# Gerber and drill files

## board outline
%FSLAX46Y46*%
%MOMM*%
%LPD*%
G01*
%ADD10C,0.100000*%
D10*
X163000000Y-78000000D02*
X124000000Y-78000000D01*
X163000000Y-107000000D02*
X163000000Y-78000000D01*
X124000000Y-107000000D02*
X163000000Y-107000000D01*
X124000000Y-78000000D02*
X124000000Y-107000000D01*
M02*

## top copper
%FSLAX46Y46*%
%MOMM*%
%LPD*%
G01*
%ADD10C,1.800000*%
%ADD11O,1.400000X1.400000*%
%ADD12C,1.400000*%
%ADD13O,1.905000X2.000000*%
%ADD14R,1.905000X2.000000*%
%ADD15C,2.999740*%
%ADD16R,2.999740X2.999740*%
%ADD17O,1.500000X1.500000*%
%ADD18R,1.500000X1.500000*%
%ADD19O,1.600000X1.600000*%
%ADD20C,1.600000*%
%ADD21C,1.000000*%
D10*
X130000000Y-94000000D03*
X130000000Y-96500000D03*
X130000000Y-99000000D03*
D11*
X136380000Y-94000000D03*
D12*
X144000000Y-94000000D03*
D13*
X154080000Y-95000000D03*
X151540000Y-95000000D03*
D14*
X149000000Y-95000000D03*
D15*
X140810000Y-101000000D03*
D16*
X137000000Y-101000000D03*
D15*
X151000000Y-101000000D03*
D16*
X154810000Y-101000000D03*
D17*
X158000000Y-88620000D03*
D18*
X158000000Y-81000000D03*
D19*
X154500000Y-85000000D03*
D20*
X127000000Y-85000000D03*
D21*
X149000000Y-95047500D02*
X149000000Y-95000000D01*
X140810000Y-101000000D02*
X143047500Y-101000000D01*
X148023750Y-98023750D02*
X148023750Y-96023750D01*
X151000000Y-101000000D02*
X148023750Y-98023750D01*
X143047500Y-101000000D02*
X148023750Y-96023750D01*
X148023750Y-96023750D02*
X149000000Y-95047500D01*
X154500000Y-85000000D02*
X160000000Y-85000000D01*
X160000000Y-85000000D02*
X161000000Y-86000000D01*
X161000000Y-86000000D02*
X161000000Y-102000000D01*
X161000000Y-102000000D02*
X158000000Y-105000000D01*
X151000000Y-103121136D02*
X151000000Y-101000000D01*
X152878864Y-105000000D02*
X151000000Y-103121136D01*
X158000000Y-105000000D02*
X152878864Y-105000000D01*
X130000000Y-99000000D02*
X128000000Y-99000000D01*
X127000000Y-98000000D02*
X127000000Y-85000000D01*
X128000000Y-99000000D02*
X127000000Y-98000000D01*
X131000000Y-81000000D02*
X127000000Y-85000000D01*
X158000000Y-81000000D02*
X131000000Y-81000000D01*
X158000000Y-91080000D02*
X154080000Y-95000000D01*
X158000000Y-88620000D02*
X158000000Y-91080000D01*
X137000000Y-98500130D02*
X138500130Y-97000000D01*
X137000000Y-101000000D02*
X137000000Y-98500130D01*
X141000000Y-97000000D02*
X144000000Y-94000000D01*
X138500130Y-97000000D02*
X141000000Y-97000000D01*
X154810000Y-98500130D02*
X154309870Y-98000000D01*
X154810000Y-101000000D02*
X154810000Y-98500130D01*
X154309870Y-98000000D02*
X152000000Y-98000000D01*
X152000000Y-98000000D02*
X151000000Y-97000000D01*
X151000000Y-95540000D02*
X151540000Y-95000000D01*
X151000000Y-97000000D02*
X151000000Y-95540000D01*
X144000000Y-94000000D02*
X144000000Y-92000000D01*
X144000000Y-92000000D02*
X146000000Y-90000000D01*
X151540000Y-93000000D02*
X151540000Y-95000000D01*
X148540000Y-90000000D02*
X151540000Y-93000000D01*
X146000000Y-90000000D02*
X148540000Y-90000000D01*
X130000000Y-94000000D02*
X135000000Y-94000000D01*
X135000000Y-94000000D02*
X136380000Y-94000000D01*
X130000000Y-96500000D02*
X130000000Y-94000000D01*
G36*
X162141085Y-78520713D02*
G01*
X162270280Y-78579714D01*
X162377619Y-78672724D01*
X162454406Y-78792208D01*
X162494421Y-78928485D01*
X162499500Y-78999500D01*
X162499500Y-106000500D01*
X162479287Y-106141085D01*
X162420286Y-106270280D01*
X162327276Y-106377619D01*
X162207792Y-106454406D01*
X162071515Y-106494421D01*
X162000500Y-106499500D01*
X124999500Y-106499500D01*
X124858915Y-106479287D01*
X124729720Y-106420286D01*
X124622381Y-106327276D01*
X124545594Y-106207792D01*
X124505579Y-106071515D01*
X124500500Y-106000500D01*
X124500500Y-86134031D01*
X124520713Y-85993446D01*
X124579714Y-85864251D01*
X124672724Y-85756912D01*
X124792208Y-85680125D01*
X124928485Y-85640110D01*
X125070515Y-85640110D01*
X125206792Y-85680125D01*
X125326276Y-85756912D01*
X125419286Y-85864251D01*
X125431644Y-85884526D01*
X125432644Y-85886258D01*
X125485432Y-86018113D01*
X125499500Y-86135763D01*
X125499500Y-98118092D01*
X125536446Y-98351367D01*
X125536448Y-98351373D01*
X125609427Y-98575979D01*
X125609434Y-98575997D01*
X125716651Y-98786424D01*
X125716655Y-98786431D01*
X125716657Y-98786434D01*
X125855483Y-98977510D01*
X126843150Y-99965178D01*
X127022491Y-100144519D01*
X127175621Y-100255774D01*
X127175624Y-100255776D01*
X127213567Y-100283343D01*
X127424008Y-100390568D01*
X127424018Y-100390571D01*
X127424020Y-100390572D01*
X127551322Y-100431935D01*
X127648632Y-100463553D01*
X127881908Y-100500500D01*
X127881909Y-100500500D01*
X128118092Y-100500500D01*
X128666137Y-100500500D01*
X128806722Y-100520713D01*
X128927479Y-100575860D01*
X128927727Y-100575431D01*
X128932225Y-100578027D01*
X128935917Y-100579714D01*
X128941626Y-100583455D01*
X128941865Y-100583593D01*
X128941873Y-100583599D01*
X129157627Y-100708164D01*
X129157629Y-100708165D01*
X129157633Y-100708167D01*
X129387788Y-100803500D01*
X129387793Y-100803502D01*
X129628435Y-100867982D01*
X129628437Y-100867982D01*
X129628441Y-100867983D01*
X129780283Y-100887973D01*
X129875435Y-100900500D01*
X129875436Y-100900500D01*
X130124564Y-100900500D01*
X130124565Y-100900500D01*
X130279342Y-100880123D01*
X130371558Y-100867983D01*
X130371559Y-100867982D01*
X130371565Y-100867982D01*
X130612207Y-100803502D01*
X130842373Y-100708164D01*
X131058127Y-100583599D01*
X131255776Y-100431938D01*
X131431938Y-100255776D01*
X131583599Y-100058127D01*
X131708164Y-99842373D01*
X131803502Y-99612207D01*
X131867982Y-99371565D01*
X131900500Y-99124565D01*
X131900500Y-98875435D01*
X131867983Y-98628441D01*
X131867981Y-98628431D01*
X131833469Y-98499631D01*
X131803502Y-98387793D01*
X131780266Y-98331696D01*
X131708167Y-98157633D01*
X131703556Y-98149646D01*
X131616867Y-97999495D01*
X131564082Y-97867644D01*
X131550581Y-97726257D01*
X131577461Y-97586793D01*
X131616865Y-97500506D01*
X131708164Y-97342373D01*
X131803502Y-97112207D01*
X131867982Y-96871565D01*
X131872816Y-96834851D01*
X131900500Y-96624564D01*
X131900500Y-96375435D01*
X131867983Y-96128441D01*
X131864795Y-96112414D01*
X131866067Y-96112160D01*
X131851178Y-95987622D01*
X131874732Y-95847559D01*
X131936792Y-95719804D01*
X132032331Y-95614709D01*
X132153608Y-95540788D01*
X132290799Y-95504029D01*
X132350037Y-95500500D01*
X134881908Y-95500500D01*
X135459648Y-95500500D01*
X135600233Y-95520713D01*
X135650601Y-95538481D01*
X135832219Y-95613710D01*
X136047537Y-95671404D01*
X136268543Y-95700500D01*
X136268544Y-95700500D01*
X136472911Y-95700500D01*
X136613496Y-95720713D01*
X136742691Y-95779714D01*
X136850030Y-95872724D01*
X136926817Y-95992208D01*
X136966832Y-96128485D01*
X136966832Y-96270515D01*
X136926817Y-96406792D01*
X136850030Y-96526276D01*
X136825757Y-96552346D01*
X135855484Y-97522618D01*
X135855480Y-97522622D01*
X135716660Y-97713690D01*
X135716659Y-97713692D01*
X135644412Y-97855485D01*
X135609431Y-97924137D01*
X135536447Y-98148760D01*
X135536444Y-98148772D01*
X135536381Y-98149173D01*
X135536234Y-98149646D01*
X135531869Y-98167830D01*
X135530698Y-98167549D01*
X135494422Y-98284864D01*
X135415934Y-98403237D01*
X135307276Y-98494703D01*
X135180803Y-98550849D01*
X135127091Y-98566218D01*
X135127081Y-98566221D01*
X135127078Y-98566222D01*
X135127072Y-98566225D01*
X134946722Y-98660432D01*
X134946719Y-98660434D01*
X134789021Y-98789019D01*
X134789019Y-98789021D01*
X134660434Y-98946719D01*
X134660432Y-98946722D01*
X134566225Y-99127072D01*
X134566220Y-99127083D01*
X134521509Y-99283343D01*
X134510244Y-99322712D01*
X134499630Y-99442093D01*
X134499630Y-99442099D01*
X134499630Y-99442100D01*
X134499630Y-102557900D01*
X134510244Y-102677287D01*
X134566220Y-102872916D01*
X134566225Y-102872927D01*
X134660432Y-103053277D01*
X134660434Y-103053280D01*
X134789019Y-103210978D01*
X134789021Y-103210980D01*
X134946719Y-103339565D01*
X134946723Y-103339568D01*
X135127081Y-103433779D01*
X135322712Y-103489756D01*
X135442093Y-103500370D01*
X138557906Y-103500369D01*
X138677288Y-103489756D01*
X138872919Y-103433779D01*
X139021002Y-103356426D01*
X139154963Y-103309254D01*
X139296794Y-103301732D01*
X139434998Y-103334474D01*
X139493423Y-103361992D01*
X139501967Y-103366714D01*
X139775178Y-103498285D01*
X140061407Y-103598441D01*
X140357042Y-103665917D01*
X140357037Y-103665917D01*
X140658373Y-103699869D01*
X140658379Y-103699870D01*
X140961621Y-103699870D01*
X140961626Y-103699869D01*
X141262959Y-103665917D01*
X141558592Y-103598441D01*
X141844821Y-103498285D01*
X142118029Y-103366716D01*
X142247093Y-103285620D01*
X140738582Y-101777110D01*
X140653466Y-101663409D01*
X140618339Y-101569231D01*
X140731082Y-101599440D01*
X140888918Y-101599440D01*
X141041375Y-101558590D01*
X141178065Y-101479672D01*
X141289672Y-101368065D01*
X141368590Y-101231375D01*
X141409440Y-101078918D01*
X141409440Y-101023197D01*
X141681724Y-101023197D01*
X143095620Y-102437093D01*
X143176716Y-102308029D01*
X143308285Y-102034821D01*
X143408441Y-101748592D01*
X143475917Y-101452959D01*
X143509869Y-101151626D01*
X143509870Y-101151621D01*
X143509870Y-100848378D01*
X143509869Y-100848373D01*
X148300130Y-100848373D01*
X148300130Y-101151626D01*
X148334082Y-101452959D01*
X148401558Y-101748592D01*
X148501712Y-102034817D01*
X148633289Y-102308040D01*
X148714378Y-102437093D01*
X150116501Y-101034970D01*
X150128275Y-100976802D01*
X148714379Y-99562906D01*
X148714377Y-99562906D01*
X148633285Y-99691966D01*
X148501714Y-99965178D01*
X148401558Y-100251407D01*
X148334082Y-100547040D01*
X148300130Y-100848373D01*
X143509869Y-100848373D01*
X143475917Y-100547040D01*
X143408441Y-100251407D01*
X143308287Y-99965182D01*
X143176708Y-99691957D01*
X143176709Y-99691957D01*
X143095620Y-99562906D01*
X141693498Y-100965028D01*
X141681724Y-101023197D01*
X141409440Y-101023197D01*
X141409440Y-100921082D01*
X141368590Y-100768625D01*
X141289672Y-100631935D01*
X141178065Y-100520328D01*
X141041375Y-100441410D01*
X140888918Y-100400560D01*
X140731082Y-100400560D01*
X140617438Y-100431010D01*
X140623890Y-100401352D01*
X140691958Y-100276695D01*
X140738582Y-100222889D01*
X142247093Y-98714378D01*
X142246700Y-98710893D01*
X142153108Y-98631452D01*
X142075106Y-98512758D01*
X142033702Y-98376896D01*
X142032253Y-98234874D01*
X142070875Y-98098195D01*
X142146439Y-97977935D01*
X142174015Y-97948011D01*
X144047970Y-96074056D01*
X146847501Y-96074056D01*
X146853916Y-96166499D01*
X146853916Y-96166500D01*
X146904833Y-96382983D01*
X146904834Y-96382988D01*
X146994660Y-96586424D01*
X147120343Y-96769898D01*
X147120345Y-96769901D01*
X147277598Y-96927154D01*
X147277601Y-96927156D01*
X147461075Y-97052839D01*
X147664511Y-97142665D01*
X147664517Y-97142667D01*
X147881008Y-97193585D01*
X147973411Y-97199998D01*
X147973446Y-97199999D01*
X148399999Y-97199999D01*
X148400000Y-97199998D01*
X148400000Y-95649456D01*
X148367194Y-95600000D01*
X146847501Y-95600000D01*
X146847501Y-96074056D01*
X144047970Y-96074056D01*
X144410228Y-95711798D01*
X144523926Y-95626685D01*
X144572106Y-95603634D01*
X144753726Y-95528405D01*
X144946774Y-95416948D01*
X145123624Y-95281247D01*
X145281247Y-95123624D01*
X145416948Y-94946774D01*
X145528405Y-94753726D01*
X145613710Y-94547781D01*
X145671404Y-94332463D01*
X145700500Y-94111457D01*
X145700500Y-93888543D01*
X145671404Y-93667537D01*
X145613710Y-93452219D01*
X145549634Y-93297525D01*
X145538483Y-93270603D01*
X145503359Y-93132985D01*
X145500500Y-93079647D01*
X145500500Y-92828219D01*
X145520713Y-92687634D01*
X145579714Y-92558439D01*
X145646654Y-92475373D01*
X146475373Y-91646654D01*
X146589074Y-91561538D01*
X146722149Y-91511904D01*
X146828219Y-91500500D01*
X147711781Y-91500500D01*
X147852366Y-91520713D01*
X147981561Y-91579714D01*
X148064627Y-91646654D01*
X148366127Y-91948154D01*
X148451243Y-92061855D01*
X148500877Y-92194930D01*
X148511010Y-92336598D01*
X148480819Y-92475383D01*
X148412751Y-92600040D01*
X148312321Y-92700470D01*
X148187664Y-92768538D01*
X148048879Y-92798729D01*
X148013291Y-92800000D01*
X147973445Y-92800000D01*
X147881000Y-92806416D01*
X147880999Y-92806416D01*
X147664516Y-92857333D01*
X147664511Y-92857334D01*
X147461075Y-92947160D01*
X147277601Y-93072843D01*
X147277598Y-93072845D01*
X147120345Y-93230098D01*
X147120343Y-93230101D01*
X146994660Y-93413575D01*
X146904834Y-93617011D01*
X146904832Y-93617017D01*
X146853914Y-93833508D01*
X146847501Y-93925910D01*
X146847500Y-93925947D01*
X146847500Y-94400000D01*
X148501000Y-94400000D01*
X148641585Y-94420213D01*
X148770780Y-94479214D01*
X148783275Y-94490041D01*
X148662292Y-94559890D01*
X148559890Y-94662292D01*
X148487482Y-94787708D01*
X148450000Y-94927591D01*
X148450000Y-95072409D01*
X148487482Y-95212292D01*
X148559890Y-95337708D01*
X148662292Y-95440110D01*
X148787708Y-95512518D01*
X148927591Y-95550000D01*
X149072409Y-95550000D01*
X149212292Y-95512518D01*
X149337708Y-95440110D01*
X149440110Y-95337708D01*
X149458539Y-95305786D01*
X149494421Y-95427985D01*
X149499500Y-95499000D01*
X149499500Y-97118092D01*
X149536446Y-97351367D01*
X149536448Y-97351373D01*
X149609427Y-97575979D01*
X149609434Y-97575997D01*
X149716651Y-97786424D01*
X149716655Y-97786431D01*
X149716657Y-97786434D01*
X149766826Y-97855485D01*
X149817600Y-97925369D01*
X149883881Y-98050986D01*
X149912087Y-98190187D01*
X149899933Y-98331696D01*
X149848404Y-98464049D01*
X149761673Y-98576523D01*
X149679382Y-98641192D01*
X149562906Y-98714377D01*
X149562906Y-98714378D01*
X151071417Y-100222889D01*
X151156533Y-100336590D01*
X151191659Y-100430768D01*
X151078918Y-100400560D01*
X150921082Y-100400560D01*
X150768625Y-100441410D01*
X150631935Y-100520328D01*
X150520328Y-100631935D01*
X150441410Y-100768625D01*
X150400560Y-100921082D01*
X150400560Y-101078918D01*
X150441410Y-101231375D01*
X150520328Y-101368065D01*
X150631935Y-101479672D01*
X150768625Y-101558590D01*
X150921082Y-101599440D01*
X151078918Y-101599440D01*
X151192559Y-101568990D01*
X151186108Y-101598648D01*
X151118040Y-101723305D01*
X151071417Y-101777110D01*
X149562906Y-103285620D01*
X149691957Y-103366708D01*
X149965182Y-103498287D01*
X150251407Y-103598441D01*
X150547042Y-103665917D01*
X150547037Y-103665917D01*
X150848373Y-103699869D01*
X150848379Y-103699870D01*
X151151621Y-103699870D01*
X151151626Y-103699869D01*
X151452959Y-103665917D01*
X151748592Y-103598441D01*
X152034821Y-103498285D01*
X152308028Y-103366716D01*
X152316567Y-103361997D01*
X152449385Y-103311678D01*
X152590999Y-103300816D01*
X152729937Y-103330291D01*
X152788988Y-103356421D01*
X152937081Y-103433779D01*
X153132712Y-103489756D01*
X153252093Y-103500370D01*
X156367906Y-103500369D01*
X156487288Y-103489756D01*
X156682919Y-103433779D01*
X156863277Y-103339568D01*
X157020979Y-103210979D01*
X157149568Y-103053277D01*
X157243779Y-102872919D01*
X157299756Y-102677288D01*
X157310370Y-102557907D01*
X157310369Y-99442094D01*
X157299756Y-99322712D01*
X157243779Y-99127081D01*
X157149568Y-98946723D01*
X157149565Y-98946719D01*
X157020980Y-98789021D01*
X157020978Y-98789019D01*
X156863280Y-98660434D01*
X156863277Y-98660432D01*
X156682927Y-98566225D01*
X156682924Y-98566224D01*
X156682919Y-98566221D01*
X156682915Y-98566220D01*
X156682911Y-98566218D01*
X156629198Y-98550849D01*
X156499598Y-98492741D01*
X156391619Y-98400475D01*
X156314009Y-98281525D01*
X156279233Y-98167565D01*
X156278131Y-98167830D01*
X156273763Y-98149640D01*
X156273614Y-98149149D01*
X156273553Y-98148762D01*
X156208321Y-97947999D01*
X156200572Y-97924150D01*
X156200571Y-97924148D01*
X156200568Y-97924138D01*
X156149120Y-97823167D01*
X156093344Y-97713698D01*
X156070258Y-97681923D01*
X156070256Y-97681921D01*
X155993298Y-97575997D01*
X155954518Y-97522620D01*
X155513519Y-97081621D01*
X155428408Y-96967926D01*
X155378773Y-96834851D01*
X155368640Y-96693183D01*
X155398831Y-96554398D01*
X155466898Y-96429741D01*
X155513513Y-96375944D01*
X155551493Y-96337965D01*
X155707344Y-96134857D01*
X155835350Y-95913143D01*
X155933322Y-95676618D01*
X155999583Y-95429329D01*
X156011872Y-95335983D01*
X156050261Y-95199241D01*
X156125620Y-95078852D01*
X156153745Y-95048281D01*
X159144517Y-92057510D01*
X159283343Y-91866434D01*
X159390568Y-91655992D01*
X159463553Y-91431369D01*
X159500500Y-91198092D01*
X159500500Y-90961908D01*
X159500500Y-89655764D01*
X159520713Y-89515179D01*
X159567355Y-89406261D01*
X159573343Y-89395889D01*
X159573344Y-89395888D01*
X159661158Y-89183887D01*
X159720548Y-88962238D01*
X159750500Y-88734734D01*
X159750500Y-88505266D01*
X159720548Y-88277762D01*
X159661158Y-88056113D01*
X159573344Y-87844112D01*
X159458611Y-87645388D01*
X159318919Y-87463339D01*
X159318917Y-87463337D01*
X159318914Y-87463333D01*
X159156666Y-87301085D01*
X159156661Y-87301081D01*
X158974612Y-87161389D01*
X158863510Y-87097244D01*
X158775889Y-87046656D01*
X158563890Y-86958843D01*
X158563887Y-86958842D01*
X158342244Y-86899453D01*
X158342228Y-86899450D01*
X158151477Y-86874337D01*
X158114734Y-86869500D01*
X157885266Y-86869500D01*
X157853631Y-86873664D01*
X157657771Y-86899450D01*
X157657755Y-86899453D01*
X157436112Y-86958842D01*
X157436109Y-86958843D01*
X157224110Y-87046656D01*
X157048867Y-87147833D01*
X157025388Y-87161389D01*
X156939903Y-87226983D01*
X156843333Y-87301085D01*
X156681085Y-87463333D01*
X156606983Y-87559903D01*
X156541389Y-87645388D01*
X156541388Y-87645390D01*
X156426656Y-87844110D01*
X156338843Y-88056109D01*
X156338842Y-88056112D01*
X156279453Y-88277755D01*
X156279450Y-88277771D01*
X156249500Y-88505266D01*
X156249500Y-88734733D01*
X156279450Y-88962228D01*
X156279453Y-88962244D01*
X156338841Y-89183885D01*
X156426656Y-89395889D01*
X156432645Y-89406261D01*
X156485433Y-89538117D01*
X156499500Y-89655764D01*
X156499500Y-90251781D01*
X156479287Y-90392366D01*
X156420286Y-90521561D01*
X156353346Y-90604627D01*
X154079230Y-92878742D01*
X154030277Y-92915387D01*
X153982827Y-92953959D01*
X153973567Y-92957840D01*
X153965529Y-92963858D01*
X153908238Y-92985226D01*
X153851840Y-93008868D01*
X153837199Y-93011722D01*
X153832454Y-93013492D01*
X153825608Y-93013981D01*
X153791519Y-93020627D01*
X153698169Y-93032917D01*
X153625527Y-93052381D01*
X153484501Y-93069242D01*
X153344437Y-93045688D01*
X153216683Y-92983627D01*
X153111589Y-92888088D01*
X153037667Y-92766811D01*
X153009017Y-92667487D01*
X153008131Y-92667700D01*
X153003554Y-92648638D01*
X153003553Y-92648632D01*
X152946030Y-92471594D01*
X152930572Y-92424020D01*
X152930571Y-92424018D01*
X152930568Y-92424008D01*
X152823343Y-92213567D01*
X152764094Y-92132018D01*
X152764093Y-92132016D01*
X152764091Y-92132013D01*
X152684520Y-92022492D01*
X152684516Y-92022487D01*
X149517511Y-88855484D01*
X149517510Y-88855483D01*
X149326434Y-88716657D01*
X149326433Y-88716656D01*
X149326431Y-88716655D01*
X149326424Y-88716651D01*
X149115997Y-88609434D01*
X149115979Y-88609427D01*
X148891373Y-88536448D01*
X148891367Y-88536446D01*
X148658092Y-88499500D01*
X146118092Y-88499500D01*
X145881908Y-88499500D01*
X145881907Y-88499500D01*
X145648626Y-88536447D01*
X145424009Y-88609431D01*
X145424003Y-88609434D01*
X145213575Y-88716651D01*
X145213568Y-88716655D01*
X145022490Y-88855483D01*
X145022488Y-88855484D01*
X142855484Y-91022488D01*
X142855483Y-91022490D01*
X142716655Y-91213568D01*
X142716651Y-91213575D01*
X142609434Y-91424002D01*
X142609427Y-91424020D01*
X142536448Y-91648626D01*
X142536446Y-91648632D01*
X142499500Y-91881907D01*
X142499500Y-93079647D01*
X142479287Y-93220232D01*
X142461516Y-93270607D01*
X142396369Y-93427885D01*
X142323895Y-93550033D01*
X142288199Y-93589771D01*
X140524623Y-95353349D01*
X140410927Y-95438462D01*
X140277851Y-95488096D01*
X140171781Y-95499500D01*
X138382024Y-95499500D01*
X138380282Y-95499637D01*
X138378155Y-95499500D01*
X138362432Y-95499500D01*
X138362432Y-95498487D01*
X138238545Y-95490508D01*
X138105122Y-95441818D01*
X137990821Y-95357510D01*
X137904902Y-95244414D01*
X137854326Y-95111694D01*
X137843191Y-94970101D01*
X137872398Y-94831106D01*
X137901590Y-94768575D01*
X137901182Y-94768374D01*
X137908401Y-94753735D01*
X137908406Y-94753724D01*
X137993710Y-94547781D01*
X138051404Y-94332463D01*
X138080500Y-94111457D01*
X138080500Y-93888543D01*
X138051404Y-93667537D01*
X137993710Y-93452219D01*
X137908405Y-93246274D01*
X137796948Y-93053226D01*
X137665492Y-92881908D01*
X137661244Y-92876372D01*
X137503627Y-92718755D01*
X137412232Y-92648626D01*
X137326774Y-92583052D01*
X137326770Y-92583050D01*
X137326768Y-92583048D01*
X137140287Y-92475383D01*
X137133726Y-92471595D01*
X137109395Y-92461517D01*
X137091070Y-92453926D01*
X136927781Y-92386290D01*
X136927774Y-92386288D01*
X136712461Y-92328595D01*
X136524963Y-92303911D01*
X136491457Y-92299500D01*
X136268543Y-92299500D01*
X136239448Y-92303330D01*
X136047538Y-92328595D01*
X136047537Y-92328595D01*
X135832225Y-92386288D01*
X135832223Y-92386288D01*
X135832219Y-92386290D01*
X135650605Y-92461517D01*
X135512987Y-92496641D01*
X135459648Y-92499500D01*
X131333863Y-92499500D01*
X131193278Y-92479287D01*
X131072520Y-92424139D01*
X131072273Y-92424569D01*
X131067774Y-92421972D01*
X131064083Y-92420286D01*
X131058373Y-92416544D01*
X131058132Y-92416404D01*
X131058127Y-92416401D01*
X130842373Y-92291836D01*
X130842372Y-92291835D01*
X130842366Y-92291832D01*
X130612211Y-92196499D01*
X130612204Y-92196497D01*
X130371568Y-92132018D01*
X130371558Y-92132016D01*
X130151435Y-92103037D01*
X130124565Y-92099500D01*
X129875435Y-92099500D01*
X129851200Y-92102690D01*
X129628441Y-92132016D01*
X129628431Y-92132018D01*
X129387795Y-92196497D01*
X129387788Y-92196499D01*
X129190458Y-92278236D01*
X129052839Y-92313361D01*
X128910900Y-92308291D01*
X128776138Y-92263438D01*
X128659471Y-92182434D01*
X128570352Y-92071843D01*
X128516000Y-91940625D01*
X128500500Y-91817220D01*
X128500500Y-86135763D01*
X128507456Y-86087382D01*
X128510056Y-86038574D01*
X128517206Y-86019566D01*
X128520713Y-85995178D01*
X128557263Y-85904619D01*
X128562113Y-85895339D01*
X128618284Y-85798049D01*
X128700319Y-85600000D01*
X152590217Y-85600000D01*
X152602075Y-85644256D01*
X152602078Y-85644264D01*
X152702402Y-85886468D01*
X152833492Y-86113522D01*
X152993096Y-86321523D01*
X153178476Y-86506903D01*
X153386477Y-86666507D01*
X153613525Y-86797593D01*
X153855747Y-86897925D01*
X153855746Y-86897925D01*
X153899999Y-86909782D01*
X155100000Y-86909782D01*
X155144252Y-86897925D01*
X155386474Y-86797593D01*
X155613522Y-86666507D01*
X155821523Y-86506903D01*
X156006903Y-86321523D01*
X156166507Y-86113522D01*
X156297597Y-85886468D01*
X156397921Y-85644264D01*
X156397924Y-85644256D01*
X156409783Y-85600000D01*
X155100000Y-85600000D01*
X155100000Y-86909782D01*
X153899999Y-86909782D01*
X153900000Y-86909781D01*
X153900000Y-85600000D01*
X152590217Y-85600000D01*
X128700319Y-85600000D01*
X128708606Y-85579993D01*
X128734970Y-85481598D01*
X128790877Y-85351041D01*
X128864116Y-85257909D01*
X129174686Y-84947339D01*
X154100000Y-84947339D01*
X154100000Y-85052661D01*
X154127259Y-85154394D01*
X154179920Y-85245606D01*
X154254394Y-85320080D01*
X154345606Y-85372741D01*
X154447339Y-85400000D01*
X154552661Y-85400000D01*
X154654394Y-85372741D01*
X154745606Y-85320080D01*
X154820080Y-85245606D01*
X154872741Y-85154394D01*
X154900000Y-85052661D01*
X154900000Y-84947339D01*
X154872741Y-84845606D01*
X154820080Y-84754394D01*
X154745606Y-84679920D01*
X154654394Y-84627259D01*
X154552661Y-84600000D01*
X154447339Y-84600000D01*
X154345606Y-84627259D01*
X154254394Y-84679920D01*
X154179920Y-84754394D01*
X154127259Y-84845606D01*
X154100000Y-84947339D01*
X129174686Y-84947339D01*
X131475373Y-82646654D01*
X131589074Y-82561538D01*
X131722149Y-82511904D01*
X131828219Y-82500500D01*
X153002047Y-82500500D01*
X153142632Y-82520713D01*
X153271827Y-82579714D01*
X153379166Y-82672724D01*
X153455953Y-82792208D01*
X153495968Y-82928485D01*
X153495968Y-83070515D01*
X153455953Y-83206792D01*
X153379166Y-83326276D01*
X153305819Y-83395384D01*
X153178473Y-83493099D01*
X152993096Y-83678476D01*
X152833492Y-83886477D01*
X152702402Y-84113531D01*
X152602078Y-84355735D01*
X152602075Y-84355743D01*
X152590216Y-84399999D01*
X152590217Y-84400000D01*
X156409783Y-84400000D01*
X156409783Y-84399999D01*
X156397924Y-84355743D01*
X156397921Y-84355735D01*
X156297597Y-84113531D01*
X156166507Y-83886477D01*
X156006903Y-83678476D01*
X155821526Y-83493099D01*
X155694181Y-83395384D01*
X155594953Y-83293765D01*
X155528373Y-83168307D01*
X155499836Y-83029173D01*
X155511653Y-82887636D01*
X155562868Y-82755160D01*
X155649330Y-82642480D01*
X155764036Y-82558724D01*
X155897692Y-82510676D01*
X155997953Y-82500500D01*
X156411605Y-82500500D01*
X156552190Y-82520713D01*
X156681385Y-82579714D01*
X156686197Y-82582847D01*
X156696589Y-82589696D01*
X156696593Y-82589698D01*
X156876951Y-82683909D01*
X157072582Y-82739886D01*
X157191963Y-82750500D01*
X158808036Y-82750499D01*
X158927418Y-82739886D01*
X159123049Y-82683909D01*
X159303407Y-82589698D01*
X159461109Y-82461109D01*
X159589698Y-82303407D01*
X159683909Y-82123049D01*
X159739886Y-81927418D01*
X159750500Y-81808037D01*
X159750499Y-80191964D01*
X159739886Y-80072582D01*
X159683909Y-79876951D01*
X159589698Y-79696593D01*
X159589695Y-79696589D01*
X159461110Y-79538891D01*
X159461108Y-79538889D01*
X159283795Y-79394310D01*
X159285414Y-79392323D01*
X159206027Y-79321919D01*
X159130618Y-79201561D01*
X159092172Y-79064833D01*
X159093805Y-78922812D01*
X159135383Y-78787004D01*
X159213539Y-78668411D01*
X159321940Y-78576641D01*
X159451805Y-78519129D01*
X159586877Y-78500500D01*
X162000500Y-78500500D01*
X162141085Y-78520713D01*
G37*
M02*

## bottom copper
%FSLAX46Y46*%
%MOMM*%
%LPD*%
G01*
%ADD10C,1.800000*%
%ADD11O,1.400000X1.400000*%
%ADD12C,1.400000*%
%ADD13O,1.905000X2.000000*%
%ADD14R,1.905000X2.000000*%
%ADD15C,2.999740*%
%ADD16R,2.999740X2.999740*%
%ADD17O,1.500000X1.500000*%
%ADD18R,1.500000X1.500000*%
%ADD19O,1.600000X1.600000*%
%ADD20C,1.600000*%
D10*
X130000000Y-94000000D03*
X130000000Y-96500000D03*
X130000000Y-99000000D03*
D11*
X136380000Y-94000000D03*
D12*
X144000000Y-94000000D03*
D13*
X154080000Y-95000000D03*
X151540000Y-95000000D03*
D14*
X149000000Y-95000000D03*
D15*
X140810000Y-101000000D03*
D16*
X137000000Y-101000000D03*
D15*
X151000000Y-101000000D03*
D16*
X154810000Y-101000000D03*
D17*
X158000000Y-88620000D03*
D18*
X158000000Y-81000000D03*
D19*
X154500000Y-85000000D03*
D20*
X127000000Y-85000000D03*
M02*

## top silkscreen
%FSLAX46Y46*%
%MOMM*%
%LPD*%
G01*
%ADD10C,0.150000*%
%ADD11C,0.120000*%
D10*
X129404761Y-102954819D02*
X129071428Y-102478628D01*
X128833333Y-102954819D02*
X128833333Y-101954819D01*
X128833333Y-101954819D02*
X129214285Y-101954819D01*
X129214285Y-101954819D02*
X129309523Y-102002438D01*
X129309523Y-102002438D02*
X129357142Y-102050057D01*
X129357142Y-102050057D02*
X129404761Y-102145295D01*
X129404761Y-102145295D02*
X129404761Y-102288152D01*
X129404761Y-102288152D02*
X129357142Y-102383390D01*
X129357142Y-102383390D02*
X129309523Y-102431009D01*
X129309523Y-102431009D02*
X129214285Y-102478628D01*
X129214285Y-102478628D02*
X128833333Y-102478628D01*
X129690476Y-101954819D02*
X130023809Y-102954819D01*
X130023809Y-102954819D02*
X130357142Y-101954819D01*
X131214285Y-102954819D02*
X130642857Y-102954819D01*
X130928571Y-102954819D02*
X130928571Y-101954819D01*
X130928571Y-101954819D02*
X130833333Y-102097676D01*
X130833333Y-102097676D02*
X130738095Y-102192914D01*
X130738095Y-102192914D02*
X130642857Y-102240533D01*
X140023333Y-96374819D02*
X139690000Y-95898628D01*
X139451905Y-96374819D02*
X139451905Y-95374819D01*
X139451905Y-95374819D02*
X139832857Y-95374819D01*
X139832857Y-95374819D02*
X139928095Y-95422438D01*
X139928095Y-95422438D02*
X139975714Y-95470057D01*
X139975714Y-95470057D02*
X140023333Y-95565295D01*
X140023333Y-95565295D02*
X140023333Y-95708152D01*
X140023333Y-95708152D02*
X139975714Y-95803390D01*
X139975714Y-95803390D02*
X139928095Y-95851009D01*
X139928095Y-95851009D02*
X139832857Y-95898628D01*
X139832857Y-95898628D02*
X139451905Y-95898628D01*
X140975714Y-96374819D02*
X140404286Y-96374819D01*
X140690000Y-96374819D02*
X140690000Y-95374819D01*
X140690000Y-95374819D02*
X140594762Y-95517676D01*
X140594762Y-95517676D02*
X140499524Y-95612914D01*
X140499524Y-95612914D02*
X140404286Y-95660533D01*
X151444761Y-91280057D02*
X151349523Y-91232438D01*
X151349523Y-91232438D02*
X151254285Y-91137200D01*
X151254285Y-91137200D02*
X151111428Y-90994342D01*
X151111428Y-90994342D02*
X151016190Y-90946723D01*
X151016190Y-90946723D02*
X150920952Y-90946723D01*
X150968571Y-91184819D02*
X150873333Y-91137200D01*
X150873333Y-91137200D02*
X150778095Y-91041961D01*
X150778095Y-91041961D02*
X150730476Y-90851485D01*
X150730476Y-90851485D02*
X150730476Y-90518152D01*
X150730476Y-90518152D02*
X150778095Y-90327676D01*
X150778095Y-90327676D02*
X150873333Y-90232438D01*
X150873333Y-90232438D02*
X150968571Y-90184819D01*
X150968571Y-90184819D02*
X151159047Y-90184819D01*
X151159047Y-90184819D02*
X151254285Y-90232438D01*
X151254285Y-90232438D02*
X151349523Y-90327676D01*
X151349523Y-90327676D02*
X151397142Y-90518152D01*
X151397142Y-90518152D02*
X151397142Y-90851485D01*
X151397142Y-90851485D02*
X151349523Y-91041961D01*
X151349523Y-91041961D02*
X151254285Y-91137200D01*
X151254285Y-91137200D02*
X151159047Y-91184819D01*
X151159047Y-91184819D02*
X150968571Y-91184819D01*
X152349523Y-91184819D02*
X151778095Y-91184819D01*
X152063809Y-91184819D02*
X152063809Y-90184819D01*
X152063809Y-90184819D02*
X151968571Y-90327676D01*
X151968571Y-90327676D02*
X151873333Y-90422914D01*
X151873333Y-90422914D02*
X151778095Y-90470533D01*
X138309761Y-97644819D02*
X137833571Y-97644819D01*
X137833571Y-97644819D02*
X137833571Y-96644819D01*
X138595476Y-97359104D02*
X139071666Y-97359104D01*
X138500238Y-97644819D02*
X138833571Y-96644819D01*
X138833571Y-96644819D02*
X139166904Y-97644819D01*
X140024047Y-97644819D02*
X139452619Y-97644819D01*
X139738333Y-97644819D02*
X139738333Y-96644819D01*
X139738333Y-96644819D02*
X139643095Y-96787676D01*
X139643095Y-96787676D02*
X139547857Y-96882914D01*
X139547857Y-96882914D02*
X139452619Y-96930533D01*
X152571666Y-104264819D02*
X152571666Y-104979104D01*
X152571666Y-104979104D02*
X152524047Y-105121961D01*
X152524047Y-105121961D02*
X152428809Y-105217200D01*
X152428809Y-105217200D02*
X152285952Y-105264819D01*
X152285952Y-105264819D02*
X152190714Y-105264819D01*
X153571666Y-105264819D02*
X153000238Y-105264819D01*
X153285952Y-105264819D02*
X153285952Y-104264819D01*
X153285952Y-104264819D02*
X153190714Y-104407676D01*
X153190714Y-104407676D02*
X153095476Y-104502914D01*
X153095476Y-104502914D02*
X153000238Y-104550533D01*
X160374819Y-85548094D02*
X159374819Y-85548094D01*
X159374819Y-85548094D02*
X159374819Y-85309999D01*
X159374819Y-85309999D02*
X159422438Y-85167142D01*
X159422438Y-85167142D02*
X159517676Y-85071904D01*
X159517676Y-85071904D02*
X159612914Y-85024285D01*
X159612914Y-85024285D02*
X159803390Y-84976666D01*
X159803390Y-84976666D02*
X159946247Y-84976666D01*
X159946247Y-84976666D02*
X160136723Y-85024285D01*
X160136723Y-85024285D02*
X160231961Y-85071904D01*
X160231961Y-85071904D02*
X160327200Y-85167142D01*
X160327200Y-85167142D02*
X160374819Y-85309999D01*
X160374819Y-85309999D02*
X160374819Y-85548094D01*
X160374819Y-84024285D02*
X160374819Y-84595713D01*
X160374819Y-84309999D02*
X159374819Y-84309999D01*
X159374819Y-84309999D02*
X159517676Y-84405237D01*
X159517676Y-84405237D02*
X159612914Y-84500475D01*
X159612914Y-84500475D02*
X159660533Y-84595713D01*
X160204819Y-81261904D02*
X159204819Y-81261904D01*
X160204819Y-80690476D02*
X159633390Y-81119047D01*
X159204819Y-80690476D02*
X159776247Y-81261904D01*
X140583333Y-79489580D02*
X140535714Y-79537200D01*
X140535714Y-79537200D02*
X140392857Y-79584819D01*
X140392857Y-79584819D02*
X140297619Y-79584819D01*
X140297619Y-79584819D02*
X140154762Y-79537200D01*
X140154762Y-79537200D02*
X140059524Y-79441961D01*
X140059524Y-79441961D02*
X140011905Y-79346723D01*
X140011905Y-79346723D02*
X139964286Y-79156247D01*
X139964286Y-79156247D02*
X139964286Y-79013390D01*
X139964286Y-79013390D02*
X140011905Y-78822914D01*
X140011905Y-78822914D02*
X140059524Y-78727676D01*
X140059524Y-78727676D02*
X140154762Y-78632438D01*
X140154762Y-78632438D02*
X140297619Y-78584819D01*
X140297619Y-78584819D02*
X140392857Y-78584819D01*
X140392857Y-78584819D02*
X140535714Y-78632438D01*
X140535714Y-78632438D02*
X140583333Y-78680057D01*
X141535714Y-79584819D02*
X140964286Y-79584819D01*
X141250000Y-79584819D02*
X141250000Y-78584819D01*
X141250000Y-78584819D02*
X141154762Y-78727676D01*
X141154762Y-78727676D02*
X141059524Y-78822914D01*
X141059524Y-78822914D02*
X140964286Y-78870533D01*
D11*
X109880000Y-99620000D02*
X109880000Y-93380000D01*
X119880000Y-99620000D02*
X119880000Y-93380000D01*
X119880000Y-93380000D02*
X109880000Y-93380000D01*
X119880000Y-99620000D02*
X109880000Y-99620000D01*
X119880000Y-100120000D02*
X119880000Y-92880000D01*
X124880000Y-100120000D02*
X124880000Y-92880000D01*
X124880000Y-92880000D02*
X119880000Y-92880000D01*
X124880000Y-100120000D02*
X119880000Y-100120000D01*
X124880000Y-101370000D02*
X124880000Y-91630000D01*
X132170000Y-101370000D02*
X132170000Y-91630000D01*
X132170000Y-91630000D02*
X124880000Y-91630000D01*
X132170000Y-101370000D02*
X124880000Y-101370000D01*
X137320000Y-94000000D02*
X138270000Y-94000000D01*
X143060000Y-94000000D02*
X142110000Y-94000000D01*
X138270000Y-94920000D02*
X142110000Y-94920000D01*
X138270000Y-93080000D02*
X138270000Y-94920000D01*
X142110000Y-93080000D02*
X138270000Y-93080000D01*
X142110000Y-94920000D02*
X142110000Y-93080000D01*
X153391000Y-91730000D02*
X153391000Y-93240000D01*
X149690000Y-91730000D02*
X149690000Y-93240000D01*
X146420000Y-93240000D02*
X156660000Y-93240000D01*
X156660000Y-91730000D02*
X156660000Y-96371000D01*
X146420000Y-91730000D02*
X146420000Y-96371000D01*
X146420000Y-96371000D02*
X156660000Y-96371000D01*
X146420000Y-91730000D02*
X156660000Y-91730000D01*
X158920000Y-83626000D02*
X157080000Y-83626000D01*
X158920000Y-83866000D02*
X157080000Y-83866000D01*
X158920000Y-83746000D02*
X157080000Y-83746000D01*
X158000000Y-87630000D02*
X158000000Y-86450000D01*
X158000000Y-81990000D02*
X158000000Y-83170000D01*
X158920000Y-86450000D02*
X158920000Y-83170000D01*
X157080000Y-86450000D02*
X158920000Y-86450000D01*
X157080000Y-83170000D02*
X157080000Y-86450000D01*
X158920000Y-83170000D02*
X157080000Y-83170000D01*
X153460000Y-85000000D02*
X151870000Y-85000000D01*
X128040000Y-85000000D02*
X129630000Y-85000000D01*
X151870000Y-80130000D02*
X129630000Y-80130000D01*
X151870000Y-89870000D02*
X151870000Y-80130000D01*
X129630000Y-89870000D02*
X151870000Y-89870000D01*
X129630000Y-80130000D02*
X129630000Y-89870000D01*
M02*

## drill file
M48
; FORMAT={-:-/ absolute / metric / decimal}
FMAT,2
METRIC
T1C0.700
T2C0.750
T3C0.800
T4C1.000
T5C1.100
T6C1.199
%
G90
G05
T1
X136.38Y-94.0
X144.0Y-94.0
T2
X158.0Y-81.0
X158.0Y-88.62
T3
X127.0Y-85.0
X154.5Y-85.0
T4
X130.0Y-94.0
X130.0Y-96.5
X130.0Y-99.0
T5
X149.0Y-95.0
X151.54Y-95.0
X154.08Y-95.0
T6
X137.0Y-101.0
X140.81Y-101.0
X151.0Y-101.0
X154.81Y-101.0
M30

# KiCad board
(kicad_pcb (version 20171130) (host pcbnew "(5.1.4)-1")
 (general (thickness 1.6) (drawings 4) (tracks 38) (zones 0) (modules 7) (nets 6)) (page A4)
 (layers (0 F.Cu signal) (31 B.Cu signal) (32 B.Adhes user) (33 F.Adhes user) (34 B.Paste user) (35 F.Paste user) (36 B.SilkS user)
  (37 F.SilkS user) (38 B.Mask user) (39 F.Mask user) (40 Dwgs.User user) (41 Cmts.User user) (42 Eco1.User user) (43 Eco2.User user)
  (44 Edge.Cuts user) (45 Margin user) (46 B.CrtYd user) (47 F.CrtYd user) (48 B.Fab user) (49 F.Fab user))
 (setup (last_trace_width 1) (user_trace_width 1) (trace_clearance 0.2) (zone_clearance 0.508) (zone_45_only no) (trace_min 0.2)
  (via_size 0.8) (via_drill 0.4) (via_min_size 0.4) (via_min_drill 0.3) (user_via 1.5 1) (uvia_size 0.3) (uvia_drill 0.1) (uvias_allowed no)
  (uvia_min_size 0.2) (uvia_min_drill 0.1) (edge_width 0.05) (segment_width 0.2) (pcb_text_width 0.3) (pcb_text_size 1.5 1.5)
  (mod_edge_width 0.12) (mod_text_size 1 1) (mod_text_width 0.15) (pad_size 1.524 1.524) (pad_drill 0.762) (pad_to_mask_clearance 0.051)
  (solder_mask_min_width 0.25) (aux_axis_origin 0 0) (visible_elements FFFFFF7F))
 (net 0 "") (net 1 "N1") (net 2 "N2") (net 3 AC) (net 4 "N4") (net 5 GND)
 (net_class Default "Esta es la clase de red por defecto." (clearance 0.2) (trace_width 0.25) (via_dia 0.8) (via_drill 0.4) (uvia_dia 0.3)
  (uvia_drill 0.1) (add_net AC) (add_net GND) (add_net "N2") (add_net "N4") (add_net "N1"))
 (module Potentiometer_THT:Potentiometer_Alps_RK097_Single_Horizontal (layer F.Cu) (at 130 94 180)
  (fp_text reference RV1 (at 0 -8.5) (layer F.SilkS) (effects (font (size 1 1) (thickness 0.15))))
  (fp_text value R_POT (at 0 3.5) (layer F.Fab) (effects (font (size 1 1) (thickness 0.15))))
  (fp_line (start 20.12 -5.62) (end 20.12 0.62) (layer F.SilkS) (width 0.12))
  (fp_line (start 10.12 -5.62) (end 10.12 0.62) (layer F.SilkS) (width 0.12))
  (fp_line (start 10.12 0.62) (end 20.12 0.62) (layer F.SilkS) (width 0.12))
  (fp_line (start 10.12 -5.62) (end 20.12 -5.62) (layer F.SilkS) (width 0.12))
  (fp_line (start 10.12 -6.12) (end 10.12 1.12) (layer F.SilkS) (width 0.12))
  (fp_line (start 5.12 -6.12) (end 5.12 1.12) (layer F.SilkS) (width 0.12))
  (fp_line (start 5.12 1.12) (end 10.12 1.12) (layer F.SilkS) (width 0.12))
  (fp_line (start 5.12 -6.12) (end 10.12 -6.12) (layer F.SilkS) (width 0.12))
  (fp_line (start 5.12 -7.37) (end 5.12 2.37) (layer F.SilkS) (width 0.12))
  (fp_line (start -2.17 -7.37) (end -2.17 2.37) (layer F.SilkS) (width 0.12))
  (fp_line (start -2.17 2.37) (end 5.12 2.37) (layer F.SilkS) (width 0.12))
  (fp_line (start -2.17 -7.37) (end 5.12 -7.37) (layer F.SilkS) (width 0.12))
  (pad 1 thru_hole circle (at 0 0 180) (size 1.8 1.8) (drill 1) (layers *.Cu *.Mask) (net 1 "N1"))
  (pad 2 thru_hole circle (at 0 -2.5 180) (size 1.8 1.8) (drill 1) (layers *.Cu *.Mask) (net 1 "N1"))
  (pad 3 thru_hole circle (at 0 -5 180) (size 1.8 1.8) (drill 1) (layers *.Cu *.Mask) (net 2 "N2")))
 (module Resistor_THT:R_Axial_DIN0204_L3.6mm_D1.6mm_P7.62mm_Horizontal (layer F.Cu) (at 144 94 180)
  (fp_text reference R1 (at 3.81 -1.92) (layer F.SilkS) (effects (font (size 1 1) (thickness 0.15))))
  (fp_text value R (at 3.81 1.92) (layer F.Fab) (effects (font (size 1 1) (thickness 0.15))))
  (fp_line (start 6.68 0) (end 5.73 0) (layer F.SilkS) (width 0.12))
  (fp_line (start 0.94 0) (end 1.89 0) (layer F.SilkS) (width 0.12))
  (fp_line (start 5.73 -0.92) (end 1.89 -0.92) (layer F.SilkS) (width 0.12))
  (fp_line (start 5.73 0.92) (end 5.73 -0.92) (layer F.SilkS) (width 0.12))
  (fp_line (start 1.89 0.92) (end 5.73 0.92) (layer F.SilkS) (width 0.12))
  (fp_line (start 1.89 -0.92) (end 1.89 0.92) (layer F.SilkS) (width 0.12))
  (pad 2 thru_hole oval (at 7.62 0 180) (size 1.4 1.4) (drill 0.7) (layers *.Cu *.Mask) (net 1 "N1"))
  (pad 1 thru_hole circle (at 0 0 180) (size 1.4 1.4) (drill 0.7) (layers *.Cu *.Mask) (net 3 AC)))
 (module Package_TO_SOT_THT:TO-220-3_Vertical (layer F.Cu) (at 149 95)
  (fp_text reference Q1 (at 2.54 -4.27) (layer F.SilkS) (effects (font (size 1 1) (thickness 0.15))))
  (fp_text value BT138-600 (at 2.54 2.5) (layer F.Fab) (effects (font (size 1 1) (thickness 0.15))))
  (fp_line (start 4.391 -3.27) (end 4.391 -1.76) (layer F.SilkS) (width 0.12))
  (fp_line (start 0.69 -3.27) (end 0.69 -1.76) (layer F.SilkS) (width 0.12))
  (fp_line (start -2.58 -1.76) (end 7.66 -1.76) (layer F.SilkS) (width 0.12))
  (fp_line (start 7.66 -3.27) (end 7.66 1.371) (layer F.SilkS) (width 0.12))
  (fp_line (start -2.58 -3.27) (end -2.58 1.371) (layer F.SilkS) (width 0.12))
  (fp_line (start -2.58 1.371) (end 7.66 1.371) (layer F.SilkS) (width 0.12))
  (fp_line (start -2.58 -3.27) (end 7.66 -3.27) (layer F.SilkS) (width 0.12))
  (pad 3 thru_hole oval (at 5.08 0) (size 1.905 2) (drill 1.1) (layers *.Cu *.Mask) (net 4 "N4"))
  (pad 2 thru_hole oval (at 2.54 0) (size 1.905 2) (drill 1.1) (layers *.Cu *.Mask) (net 3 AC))
  (pad 1 thru_hole rect (at 0 0) (size 1.905 2) (drill 1.1) (layers *.Cu *.Mask) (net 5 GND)))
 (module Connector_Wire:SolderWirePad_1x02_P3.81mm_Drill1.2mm (layer F.Cu) (at 137 101)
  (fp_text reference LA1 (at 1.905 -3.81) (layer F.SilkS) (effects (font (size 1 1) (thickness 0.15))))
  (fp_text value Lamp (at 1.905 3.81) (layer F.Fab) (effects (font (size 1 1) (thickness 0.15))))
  (pad 2 thru_hole circle (at 3.81 0) (size 2.99974 2.99974) (drill 1.19888) (layers *.Cu *.Mask) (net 5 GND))
  (pad 1 thru_hole rect (at 0 0) (size 2.99974 2.99974) (drill 1.19888) (layers *.Cu *.Mask) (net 3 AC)))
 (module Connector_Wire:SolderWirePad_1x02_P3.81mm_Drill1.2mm (layer F.Cu) (at 154.81 101 180)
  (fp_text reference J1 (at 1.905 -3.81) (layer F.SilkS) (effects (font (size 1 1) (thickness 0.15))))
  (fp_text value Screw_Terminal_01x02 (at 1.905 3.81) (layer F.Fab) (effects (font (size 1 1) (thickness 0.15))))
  (pad 2 thru_hole circle (at 3.81 0 180) (size 2.99974 2.99974) (drill 1.19888) (layers *.Cu *.Mask) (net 5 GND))
  (pad 1 thru_hole rect (at 0 0 180) (size 2.99974 2.99974) (drill 1.19888) (layers *.Cu *.Mask) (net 3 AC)))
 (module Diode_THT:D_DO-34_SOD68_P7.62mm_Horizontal (layer F.Cu) (at 158 81 270)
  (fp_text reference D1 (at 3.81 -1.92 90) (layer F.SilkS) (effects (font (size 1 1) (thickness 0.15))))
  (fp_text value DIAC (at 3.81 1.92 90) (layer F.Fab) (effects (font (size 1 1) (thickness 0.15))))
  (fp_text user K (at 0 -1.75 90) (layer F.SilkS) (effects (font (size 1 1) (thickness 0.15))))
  (fp_line (start 2.626 -0.92) (end 2.626 0.92) (layer F.SilkS) (width 0.12))
  (fp_line (start 2.866 -0.92) (end 2.866 0.92) (layer F.SilkS) (width 0.12))
  (fp_line (start 2.746 -0.92) (end 2.746 0.92) (layer F.SilkS) (width 0.12))
  (fp_line (start 6.63 0) (end 5.45 0) (layer F.SilkS) (width 0.12))
  (fp_line (start 0.99 0) (end 2.17 0) (layer F.SilkS) (width 0.12))
  (fp_line (start 5.45 -0.92) (end 2.17 -0.92) (layer F.SilkS) (width 0.12))
  (fp_line (start 5.45 0.92) (end 5.45 -0.92) (layer F.SilkS) (width 0.12))
  (fp_line (start 2.17 0.92) (end 5.45 0.92) (layer F.SilkS) (width 0.12))
  (fp_line (start 2.17 -0.92) (end 2.17 0.92) (layer F.SilkS) (width 0.12))
  (pad 2 thru_hole oval (at 7.62 0 270) (size 1.5 1.5) (drill 0.75) (layers *.Cu *.Mask) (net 4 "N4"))
  (pad 1 thru_hole rect (at 0 0 270) (size 1.5 1.5) (drill 0.75) (layers *.Cu *.Mask) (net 2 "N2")))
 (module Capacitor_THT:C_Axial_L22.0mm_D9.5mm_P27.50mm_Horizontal (layer F.Cu) (at 127 85)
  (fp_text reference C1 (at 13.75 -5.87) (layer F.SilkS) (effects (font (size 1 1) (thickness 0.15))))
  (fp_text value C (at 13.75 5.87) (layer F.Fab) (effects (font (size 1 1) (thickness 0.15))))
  (fp_line (start 26.46 0) (end 24.87 0) (layer F.SilkS) (width 0.12))
  (fp_line (start 1.04 0) (end 2.63 0) (layer F.SilkS) (width 0.12))
  (fp_line (start 24.87 -4.87) (end 2.63 -4.87) (layer F.SilkS) (width 0.12))
  (fp_line (start 24.87 4.87) (end 24.87 -4.87) (layer F.SilkS) (width 0.12))
  (fp_line (start 2.63 4.87) (end 24.87 4.87) (layer F.SilkS) (width 0.12))
  (fp_line (start 2.63 -4.87) (end 2.63 4.87) (layer F.SilkS) (width 0.12))
  (pad 2 thru_hole oval (at 27.5 0) (size 1.6 1.6) (drill 0.8) (layers *.Cu *.Mask) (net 5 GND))
  (pad 1 thru_hole circle (at 0 0) (size 1.6 1.6) (drill 0.8) (layers *.Cu *.Mask) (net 2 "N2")))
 (gr_line (start 163 78) (end 124 78) (layer Edge.Cuts) (width 0.1))
 (gr_line (start 163 107) (end 163 78) (layer Edge.Cuts) (width 0.1))
 (gr_line (start 124 107) (end 163 107) (layer Edge.Cuts) (width 0.1))
 (gr_line (start 124 78) (end 124 107) (layer Edge.Cuts) (width 0.1))
 (segment (start 149 95.0475) (end 149 95) (width 1) (layer F.Cu) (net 5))
 (segment (start 140.81 101) (end 143.0475 101) (width 1) (layer F.Cu) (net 5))
 (segment (start 148.02375 98.02375) (end 148.02375 96.02375) (width 1) (layer F.Cu) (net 5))
 (segment (start 151 101) (end 148.02375 98.02375) (width 1) (layer F.Cu) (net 5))
 (segment (start 143.0475 101) (end 148.02375 96.02375) (width 1) (layer F.Cu) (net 5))
 (segment (start 148.02375 96.02375) (end 149 95.0475) (width 1) (layer F.Cu) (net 5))
 (segment (start 154.5 85) (end 160 85) (width 1) (layer F.Cu) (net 5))
 (segment (start 160 85) (end 161 86) (width 1) (layer F.Cu) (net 5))
 (segment (start 161 86) (end 161 102) (width 1) (layer F.Cu) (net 5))
 (segment (start 161 102) (end 158 105) (width 1) (layer F.Cu) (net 5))
 (segment (start 151 103.121136) (end 151 101) (width 1) (layer F.Cu) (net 5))
 (segment (start 152.878864 105) (end 151 103.121136) (width 1) (layer F.Cu) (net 5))
 (segment (start 158 105) (end 152.878864 105) (width 1) (layer F.Cu) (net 5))
 (segment (start 130 99) (end 128 99) (width 1) (layer F.Cu) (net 2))
 (segment (start 127 98) (end 127 85) (width 1) (layer F.Cu) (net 2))
 (segment (start 128 99) (end 127 98) (width 1) (layer F.Cu) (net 2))
 (segment (start 131 81) (end 127 85) (width 1) (layer F.Cu) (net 2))
 (segment (start 158 81) (end 131 81) (width 1) (layer F.Cu) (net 2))
 (segment (start 158 91.08) (end 154.08 95) (width 1) (layer F.Cu) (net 4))
 (segment (start 158 88.62) (end 158 91.08) (width 1) (layer F.Cu) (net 4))
 (segment (start 137 98.50013) (end 138.50013 97) (width 1) (layer F.Cu) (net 3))
 (segment (start 137 101) (end 137 98.50013) (width 1) (layer F.Cu) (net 3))
 (segment (start 141 97) (end 144 94) (width 1) (layer F.Cu) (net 3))
 (segment (start 138.50013 97) (end 141 97) (width 1) (layer F.Cu) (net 3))
 (segment (start 154.81 98.50013) (end 154.30987 98) (width 1) (layer F.Cu) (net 3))
 (segment (start 154.81 101) (end 154.81 98.50013) (width 1) (layer F.Cu) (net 3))
 (segment (start 154.30987 98) (end 152 98) (width 1) (layer F.Cu) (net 3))
 (segment (start 152 98) (end 151 97) (width 1) (layer F.Cu) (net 3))
 (segment (start 151 95.54) (end 151.54 95) (width 1) (layer F.Cu) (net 3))
 (segment (start 151 97) (end 151 95.54) (width 1) (layer F.Cu) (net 3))
 (segment (start 144 94) (end 144 92) (width 1) (layer F.Cu) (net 3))
 (segment (start 144 92) (end 146 90) (width 1) (layer F.Cu) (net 3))
 (segment (start 151.54 93) (end 151.54 95) (width 1) (layer F.Cu) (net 3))
 (segment (start 148.54 90) (end 151.54 93) (width 1) (layer F.Cu) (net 3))
 (segment (start 146 90) (end 148.54 90) (width 1) (layer F.Cu) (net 3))
 (segment (start 130 94) (end 135 94) (width 1) (layer F.Cu) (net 1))
 (segment (start 135 94) (end 136.38 94) (width 1) (layer F.Cu) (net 1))
 (segment (start 130 96.5) (end 130 94) (width 1) (layer F.Cu) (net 1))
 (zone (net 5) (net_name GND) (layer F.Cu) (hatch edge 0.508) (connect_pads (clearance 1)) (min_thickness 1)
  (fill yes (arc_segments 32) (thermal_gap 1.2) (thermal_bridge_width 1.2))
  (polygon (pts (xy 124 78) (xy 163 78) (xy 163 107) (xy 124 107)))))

